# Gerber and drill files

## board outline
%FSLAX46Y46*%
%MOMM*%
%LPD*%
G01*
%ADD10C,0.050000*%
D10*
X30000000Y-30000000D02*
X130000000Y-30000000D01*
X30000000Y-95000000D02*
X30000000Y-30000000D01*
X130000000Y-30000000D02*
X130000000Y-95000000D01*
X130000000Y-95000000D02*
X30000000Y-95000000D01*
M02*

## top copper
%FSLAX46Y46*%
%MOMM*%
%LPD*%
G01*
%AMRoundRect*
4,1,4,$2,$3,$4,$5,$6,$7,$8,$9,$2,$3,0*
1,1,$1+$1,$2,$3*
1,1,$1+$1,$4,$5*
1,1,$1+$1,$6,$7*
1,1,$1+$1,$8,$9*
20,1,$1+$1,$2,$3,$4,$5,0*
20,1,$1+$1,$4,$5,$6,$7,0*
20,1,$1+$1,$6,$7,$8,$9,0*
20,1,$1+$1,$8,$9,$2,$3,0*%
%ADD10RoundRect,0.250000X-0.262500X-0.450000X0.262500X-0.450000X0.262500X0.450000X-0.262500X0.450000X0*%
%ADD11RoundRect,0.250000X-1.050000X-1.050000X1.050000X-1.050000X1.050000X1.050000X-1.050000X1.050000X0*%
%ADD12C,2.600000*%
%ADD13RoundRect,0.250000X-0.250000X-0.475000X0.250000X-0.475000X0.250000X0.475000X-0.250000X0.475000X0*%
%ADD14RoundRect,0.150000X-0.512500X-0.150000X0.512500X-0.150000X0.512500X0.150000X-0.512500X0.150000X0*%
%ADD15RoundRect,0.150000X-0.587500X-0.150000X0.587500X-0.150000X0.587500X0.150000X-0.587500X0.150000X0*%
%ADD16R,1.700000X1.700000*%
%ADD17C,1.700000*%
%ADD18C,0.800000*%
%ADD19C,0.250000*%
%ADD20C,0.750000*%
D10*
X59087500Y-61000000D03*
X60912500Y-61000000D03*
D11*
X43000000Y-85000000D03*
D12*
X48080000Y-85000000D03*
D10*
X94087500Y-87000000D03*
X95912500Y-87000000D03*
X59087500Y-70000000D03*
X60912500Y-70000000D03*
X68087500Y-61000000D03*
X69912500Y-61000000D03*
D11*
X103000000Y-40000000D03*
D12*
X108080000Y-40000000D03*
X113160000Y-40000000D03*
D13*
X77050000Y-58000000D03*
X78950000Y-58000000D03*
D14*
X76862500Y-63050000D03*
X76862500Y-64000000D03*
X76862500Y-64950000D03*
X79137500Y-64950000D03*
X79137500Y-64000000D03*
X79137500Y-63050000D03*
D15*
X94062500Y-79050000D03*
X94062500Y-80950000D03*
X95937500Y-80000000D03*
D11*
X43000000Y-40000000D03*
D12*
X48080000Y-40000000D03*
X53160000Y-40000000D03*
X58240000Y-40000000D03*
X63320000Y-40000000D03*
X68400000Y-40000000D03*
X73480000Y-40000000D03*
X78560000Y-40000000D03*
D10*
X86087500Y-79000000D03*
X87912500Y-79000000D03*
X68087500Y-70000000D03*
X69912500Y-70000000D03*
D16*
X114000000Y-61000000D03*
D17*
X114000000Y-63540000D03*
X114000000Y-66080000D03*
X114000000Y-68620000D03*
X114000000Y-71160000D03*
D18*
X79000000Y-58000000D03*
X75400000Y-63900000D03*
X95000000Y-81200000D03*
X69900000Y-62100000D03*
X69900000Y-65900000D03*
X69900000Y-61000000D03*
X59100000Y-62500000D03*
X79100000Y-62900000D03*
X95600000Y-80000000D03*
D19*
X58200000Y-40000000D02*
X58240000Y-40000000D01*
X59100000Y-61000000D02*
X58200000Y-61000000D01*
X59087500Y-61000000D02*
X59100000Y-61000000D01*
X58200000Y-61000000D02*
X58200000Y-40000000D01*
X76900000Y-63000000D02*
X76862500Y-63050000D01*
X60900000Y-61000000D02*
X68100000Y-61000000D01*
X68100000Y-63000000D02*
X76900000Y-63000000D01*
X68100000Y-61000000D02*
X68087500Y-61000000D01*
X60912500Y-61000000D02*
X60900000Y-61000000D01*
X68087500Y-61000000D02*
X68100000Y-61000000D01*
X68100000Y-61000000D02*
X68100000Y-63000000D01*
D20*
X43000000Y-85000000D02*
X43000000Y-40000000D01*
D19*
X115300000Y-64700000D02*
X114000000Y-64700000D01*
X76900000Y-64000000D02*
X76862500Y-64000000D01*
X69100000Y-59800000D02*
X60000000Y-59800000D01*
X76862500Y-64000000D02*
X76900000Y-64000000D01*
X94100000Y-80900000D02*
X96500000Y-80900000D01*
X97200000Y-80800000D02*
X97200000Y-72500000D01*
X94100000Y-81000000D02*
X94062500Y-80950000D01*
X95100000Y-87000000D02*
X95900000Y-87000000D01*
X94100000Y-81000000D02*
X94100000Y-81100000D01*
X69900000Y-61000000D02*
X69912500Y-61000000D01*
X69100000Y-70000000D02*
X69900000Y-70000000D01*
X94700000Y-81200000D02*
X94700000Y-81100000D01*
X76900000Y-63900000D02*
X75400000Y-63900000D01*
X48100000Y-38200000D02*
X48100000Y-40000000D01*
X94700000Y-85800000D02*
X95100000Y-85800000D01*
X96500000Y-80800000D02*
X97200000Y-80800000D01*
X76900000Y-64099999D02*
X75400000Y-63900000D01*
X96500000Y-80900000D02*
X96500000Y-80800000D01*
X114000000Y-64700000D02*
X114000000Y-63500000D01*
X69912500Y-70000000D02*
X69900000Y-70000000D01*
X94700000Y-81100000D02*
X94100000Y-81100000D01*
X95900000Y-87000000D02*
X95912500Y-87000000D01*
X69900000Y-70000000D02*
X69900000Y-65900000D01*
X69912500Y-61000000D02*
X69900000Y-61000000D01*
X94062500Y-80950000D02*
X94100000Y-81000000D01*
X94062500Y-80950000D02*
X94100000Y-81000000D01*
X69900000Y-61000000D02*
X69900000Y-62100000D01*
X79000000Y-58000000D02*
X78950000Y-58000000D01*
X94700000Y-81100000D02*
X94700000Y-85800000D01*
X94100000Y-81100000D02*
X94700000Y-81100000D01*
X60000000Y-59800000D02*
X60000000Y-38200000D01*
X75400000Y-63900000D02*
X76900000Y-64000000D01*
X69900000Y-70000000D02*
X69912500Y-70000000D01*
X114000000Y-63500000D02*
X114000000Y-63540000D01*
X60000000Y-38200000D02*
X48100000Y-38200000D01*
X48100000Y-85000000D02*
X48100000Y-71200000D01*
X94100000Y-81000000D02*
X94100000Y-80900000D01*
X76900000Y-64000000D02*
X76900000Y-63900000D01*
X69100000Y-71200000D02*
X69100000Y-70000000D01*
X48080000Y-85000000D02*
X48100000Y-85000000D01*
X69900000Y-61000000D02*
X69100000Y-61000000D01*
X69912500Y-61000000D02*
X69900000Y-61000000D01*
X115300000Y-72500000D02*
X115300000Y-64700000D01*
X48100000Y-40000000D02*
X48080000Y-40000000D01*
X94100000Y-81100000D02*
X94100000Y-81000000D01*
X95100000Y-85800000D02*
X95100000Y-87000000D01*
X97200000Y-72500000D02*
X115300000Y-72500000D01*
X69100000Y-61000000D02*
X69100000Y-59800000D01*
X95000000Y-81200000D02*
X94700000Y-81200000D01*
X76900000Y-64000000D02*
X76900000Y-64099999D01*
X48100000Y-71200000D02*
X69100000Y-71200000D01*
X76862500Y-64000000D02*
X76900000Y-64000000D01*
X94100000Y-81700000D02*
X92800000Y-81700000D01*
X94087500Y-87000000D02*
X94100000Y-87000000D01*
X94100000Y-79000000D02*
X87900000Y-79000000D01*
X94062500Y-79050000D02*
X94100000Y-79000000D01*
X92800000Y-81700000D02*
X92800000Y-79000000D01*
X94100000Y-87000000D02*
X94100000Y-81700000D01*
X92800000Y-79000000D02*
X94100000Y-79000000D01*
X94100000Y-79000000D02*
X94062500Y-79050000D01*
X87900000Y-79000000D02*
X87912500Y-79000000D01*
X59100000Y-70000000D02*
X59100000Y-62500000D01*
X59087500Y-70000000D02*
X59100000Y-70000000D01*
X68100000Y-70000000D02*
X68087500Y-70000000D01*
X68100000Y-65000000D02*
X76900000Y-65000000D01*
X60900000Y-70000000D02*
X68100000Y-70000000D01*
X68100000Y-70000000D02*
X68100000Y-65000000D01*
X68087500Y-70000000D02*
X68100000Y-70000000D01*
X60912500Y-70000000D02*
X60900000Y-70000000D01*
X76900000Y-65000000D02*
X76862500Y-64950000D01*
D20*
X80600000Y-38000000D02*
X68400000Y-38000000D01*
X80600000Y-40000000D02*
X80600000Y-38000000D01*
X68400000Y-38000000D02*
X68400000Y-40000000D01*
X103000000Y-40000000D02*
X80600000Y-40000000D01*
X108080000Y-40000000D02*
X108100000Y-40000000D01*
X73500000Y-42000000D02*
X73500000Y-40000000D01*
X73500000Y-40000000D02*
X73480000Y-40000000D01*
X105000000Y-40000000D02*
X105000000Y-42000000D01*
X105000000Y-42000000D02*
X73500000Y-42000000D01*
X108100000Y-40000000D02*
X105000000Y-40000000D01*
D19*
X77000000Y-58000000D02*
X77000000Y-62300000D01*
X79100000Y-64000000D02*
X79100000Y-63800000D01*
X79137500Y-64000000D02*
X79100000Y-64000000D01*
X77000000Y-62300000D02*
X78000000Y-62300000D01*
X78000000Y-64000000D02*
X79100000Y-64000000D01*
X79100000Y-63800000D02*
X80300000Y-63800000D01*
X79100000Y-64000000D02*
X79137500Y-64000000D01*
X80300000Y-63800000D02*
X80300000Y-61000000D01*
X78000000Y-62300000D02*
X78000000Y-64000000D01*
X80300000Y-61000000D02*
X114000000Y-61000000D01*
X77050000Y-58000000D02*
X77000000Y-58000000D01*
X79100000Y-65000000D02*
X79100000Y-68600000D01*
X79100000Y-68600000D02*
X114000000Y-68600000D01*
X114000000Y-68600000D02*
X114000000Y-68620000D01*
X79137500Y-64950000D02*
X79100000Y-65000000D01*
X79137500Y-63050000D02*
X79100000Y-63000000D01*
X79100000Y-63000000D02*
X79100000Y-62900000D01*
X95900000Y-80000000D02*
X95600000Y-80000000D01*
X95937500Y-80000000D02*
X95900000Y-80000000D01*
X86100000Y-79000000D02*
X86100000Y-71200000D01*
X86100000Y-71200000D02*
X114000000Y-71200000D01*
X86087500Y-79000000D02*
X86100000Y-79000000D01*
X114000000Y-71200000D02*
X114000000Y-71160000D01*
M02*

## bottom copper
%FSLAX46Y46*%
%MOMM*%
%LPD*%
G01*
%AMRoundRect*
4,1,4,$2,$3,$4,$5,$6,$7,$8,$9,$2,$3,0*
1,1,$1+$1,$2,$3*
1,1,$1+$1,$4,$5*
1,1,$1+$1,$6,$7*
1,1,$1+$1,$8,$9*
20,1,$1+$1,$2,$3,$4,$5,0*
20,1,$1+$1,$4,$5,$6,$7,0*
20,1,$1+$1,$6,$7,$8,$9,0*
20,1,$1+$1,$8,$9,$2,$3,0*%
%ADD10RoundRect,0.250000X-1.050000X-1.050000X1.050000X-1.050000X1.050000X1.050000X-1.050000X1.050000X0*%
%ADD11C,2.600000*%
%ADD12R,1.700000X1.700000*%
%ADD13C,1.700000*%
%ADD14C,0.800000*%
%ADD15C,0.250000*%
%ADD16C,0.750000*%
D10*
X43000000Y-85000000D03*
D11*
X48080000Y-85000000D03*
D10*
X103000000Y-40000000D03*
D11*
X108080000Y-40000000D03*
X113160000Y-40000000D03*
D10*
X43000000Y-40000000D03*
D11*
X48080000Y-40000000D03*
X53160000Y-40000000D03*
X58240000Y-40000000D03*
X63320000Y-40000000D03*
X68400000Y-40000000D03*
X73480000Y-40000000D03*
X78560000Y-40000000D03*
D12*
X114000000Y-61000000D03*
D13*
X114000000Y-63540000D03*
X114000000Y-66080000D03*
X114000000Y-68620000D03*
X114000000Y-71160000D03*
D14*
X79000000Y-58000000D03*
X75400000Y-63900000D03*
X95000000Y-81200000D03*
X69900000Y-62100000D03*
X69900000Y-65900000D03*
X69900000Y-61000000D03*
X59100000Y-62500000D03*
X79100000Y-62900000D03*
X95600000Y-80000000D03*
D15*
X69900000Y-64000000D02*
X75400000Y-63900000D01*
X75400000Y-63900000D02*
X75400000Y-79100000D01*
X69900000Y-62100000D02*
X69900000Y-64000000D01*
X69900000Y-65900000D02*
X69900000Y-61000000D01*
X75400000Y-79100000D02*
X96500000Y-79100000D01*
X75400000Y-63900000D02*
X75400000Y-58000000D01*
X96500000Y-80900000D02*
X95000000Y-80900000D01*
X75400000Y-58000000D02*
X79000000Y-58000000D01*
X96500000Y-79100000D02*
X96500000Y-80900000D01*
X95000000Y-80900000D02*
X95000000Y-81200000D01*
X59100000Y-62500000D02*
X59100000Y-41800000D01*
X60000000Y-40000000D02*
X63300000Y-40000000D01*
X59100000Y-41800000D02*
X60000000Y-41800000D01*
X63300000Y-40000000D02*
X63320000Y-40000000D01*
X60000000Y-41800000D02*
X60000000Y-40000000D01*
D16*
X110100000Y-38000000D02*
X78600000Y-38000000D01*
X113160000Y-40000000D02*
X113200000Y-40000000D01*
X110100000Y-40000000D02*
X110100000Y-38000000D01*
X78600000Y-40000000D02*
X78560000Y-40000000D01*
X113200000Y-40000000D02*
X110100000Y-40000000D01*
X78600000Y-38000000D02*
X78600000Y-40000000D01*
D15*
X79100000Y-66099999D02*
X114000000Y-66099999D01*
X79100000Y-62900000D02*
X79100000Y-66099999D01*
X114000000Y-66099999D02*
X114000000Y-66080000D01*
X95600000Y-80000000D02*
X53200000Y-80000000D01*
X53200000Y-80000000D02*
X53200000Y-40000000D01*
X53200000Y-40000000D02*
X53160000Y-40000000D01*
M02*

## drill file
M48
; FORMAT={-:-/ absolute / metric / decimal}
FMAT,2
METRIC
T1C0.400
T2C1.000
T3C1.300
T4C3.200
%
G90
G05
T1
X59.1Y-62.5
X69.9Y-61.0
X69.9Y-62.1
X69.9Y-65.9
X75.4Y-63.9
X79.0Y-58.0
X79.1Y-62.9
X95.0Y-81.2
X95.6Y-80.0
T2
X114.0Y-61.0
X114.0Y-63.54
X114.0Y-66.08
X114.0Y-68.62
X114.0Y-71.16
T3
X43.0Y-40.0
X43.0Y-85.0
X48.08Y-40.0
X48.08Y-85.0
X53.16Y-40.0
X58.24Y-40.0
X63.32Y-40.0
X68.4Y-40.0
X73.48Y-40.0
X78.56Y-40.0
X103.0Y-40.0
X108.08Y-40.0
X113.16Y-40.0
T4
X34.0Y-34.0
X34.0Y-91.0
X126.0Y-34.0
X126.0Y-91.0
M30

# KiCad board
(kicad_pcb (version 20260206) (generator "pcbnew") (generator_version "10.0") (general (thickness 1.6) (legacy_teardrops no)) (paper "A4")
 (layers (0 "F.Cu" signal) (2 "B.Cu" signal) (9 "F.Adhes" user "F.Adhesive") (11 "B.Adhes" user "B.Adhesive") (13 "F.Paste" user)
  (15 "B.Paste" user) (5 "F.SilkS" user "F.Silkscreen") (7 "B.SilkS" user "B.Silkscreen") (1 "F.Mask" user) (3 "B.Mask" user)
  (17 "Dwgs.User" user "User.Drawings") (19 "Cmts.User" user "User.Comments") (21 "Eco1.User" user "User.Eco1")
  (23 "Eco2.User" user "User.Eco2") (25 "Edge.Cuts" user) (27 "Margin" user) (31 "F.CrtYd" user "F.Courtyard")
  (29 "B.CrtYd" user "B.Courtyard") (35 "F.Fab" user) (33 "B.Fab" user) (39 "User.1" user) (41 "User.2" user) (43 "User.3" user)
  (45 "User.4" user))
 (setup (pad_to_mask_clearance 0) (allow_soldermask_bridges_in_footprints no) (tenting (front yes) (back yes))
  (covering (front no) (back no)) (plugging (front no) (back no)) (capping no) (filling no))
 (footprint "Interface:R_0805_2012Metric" (layer "F.Cu") (at 60 61)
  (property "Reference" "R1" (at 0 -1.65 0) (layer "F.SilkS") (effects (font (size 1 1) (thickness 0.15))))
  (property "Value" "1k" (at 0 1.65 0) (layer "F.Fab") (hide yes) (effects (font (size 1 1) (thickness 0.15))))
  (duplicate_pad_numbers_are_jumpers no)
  (pad "1" smd roundrect (at -0.9125 0) (size 1.025 1.4) (layers "F.Cu" "F.Mask" "F.Paste") (roundrect_rratio 0.243902) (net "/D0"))
  (pad "2" smd roundrect (at 0.9125 0) (size 1.025 1.4) (layers "F.Cu" "F.Mask" "F.Paste") (roundrect_rratio 0.243902) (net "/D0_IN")))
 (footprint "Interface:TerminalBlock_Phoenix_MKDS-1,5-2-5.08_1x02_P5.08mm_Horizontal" (layer "F.Cu") (at 43 85)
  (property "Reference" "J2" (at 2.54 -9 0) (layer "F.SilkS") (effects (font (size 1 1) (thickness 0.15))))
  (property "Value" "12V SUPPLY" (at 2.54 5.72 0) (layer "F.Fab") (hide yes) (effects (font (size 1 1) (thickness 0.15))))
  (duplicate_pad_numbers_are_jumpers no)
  (pad "1" thru_hole roundrect (at 0 0) (size 2.6 2.6) (drill 1.3) (layers "*.Cu" "*.Mask") (remove_unused_layers no)
   (roundrect_rratio 0.096154) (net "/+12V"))
  (pad "2" thru_hole circle (at 5.08 0) (size 2.6 2.6) (drill 1.3) (layers "*.Cu" "*.Mask") (remove_unused_layers no) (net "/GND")))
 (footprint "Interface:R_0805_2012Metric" (layer "F.Cu") (at 95 87)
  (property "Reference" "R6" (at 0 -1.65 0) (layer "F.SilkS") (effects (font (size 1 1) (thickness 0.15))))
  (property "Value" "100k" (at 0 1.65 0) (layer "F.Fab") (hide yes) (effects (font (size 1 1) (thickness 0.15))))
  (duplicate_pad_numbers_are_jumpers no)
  (pad "1" smd roundrect (at -0.9125 0) (size 1.025 1.4) (layers "F.Cu" "F.Mask" "F.Paste") (roundrect_rratio 0.243902) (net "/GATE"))
  (pad "2" smd roundrect (at 0.9125 0) (size 1.025 1.4) (layers "F.Cu" "F.Mask" "F.Paste") (roundrect_rratio 0.243902) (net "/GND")))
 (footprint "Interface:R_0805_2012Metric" (layer "F.Cu") (at 60 70)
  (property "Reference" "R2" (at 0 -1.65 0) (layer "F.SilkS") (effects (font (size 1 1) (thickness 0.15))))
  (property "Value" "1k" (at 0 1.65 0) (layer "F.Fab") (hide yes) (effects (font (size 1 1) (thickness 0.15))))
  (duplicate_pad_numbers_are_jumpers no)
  (pad "1" smd roundrect (at -0.9125 0) (size 1.025 1.4) (layers "F.Cu" "F.Mask" "F.Paste") (roundrect_rratio 0.243902) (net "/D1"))
  (pad "2" smd roundrect (at 0.9125 0) (size 1.025 1.4) (layers "F.Cu" "F.Mask" "F.Paste") (roundrect_rratio 0.243902) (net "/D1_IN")))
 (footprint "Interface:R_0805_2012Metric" (layer "F.Cu") (at 69 61)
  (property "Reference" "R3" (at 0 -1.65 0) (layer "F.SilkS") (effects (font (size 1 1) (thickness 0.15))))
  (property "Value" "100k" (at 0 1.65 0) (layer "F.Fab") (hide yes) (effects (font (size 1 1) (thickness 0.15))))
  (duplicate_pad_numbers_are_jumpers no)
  (pad "1" smd roundrect (at -0.9125 0) (size 1.025 1.4) (layers "F.Cu" "F.Mask" "F.Paste") (roundrect_rratio 0.243902) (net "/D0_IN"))
  (pad "2" smd roundrect (at 0.9125 0) (size 1.025 1.4) (layers "F.Cu" "F.Mask" "F.Paste") (roundrect_rratio 0.243902) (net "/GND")))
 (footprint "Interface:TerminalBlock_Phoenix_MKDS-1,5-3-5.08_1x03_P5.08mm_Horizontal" (layer "F.Cu") (at 103 40)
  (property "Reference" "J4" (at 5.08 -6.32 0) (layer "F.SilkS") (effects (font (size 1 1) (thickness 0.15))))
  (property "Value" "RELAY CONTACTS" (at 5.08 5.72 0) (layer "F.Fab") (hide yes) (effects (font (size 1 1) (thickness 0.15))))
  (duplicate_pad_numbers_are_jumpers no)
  (pad "1" thru_hole roundrect (at 0 0) (size 2.6 2.6) (drill 1.3) (layers "*.Cu" "*.Mask") (remove_unused_layers no)
   (roundrect_rratio 0.096154) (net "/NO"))
  (pad "2" thru_hole circle (at 5.08 0) (size 2.6 2.6) (drill 1.3) (layers "*.Cu" "*.Mask") (remove_unused_layers no) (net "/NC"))
  (pad "3" thru_hole circle (at 10.16 0) (size 2.6 2.6) (drill 1.3) (layers "*.Cu" "*.Mask") (remove_unused_layers no) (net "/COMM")))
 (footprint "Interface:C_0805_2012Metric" (layer "F.Cu") (at 78 58)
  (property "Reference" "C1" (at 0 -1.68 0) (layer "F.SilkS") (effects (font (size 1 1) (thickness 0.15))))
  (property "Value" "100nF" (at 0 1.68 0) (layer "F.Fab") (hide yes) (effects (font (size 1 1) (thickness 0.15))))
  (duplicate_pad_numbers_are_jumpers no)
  (pad "1" smd roundrect (at -0.95 0) (size 1 1.45) (layers "F.Cu" "F.Mask" "F.Paste") (roundrect_rratio 0.25) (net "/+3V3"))
  (pad "2" smd roundrect (at 0.95 0) (size 1 1.45) (layers "F.Cu" "F.Mask" "F.Paste") (roundrect_rratio 0.25) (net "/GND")))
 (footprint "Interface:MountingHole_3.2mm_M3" (layer "F.Cu") (at 34 91)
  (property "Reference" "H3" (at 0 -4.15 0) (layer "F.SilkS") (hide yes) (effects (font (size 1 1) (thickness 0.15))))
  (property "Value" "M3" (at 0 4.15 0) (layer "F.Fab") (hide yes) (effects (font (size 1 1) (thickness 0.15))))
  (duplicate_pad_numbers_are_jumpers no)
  (pad "" np_thru_hole circle (at 0 0) (size 3.2 3.2) (drill 3.2) (layers "*.Cu" "*.Mask")))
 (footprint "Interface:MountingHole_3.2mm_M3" (layer "F.Cu") (at 126 91)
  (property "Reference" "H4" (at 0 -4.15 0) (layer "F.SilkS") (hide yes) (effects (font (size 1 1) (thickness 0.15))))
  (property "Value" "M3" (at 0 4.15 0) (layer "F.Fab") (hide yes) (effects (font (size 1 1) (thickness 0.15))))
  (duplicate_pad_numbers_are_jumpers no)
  (pad "" np_thru_hole circle (at 0 0) (size 3.2 3.2) (drill 3.2) (layers "*.Cu" "*.Mask")))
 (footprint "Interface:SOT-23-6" (layer "F.Cu") (at 78 64)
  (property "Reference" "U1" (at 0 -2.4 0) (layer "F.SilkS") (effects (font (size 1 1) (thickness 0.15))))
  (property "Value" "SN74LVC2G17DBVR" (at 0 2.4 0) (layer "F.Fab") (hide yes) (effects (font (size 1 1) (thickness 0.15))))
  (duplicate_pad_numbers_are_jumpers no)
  (pad "1" smd roundrect (at -1.1375 -0.95) (size 1.325 0.6) (layers "F.Cu" "F.Mask" "F.Paste") (roundrect_rratio 0.25) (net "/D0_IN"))
  (pad "2" smd roundrect (at -1.1375 0) (size 1.325 0.6) (layers "F.Cu" "F.Mask" "F.Paste") (roundrect_rratio 0.25) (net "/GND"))
  (pad "3" smd roundrect (at -1.1375 0.95) (size 1.325 0.6) (layers "F.Cu" "F.Mask" "F.Paste") (roundrect_rratio 0.25) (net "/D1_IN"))
  (pad "4" smd roundrect (at 1.1375 0.95) (size 1.325 0.6) (layers "F.Cu" "F.Mask" "F.Paste") (roundrect_rratio 0.25) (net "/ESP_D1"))
  (pad "5" smd roundrect (at 1.1375 0) (size 1.325 0.6) (layers "F.Cu" "F.Mask" "F.Paste") (roundrect_rratio 0.25) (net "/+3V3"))
  (pad "6" smd roundrect (at 1.1375 -0.95) (size 1.325 0.6) (layers "F.Cu" "F.Mask" "F.Paste") (roundrect_rratio 0.25) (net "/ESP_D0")))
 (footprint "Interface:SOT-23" (layer "F.Cu") (at 95 80)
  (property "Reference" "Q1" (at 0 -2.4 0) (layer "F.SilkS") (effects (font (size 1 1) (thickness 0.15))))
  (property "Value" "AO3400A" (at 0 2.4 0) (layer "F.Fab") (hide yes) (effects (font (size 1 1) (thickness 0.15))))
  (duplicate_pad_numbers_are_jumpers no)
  (pad "1" smd roundrect (at -0.9375 -0.95) (size 1.475 0.6) (layers "F.Cu" "F.Mask" "F.Paste") (roundrect_rratio 0.25) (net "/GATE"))
  (pad "2" smd roundrect (at -0.9375 0.95) (size 1.475 0.6) (layers "F.Cu" "F.Mask" "F.Paste") (roundrect_rratio 0.25) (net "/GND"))
  (pad "3" smd roundrect (at 0.9375 0) (size 1.475 0.6) (layers "F.Cu" "F.Mask" "F.Paste") (roundrect_rratio 0.25) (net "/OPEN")))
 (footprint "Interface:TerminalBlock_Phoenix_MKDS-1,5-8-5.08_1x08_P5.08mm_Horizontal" (layer "F.Cu") (at 43 40)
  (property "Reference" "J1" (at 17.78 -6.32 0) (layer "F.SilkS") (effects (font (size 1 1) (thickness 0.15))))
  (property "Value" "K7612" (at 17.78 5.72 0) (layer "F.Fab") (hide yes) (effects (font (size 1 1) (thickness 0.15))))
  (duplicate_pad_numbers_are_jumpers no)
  (pad "1" thru_hole roundrect (at 0 0) (size 2.6 2.6) (drill 1.3) (layers "*.Cu" "*.Mask") (remove_unused_layers no)
   (roundrect_rratio 0.096154) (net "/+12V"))
  (pad "2" thru_hole circle (at 5.08 0) (size 2.6 2.6) (drill 1.3) (layers "*.Cu" "*.Mask") (remove_unused_layers no) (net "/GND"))
  (pad "3" thru_hole circle (at 10.16 0) (size 2.6 2.6) (drill 1.3) (layers "*.Cu" "*.Mask") (remove_unused_layers no) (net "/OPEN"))
  (pad "4" thru_hole circle (at 15.24 0) (size 2.6 2.6) (drill 1.3) (layers "*.Cu" "*.Mask") (remove_unused_layers no) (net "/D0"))
  (pad "5" thru_hole circle (at 20.32 0) (size 2.6 2.6) (drill 1.3) (layers "*.Cu" "*.Mask") (remove_unused_layers no) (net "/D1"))
  (pad "6" thru_hole circle (at 25.4 0) (size 2.6 2.6) (drill 1.3) (layers "*.Cu" "*.Mask") (remove_unused_layers no) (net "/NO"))
  (pad "7" thru_hole circle (at 30.48 0) (size 2.6 2.6) (drill 1.3) (layers "*.Cu" "*.Mask") (remove_unused_layers no) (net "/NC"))
  (pad "8" thru_hole circle (at 35.56 0) (size 2.6 2.6) (drill 1.3) (layers "*.Cu" "*.Mask") (remove_unused_layers no) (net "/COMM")))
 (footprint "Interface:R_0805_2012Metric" (layer "F.Cu") (at 87 79)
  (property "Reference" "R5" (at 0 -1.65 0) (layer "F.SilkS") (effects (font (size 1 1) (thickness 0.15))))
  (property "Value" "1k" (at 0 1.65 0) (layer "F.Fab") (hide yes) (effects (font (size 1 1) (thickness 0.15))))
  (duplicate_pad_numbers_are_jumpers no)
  (pad "1" smd roundrect (at -0.9125 0) (size 1.025 1.4) (layers "F.Cu" "F.Mask" "F.Paste") (roundrect_rratio 0.243902) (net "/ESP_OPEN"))
  (pad "2" smd roundrect (at 0.9125 0) (size 1.025 1.4) (layers "F.Cu" "F.Mask" "F.Paste") (roundrect_rratio 0.243902) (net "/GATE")))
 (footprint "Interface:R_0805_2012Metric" (layer "F.Cu") (at 69 70)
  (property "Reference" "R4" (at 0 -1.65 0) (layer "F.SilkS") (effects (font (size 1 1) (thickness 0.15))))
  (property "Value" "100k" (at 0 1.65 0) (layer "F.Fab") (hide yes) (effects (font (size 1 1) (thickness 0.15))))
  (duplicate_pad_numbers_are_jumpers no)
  (pad "1" smd roundrect (at -0.9125 0) (size 1.025 1.4) (layers "F.Cu" "F.Mask" "F.Paste") (roundrect_rratio 0.243902) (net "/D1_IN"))
  (pad "2" smd roundrect (at 0.9125 0) (size 1.025 1.4) (layers "F.Cu" "F.Mask" "F.Paste") (roundrect_rratio 0.243902) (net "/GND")))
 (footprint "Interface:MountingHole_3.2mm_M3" (layer "F.Cu") (at 126 34)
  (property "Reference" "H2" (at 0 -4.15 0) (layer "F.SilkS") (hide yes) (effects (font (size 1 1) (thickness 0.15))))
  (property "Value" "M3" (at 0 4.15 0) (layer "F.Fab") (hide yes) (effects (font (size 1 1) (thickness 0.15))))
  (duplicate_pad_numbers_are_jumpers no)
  (pad "" np_thru_hole circle (at 0 0) (size 3.2 3.2) (drill 3.2) (layers "*.Cu" "*.Mask")))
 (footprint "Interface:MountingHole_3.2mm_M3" (layer "F.Cu") (at 34 34)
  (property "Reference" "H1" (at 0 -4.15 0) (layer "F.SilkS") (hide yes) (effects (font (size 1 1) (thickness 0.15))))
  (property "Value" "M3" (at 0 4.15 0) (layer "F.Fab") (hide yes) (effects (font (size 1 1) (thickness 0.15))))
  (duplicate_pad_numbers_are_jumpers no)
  (pad "" np_thru_hole circle (at 0 0) (size 3.2 3.2) (drill 3.2) (layers "*.Cu" "*.Mask")))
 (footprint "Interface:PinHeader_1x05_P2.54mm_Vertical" (layer "F.Cu") (at 114 61)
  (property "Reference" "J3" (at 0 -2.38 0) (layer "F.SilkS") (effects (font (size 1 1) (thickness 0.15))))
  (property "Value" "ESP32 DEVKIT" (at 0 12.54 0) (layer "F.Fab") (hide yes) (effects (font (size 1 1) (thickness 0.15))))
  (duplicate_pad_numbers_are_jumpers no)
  (pad "1" thru_hole rect (at 0 0) (size 1.7 1.7) (drill 1) (layers "*.Cu" "*.Mask") (remove_unused_layers no) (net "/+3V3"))
  (pad "2" thru_hole circle (at 0 2.54) (size 1.7 1.7) (drill 1) (layers "*.Cu" "*.Mask") (remove_unused_layers no) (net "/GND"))
  (pad "3" thru_hole circle (at 0 5.08) (size 1.7 1.7) (drill 1) (layers "*.Cu" "*.Mask") (remove_unused_layers no) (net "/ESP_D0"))
  (pad "4" thru_hole circle (at 0 7.62) (size 1.7 1.7) (drill 1) (layers "*.Cu" "*.Mask") (remove_unused_layers no) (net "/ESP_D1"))
  (pad "5" thru_hole circle (at 0 10.16) (size 1.7 1.7) (drill 1) (layers "*.Cu" "*.Mask") (remove_unused_layers no) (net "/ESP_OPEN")))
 (gr_line (start 30 30) (end 130 30) (stroke (width 0.05) (type default)) (layer "Edge.Cuts"))
 (gr_line (start 30 95) (end 30 30) (stroke (width 0.05) (type default)) (layer "Edge.Cuts"))
 (gr_line (start 130 30) (end 130 95) (stroke (width 0.05) (type default)) (layer "Edge.Cuts"))
 (gr_line (start 130 95) (end 30 95) (stroke (width 0.05) (type default)) (layer "Edge.Cuts"))
 (segment (start 58.2 40) (end 58.24 40) (width 0.25) (layer "F.Cu") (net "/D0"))
 (segment (start 59.1 61) (end 58.2 61) (width 0.25) (layer "F.Cu") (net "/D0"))
 (segment (start 59.0875 61) (end 59.1 61) (width 0.25) (layer "F.Cu") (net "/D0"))
 (segment (start 58.2 61) (end 58.2 40) (width 0.25) (layer "F.Cu") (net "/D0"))
 (segment (start 76.9 63) (end 76.8625 63.05) (width 0.25) (layer "F.Cu") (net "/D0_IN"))
 (segment (start 60.9 61) (end 68.1 61) (width 0.25) (layer "F.Cu") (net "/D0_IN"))
 (segment (start 68.1 63) (end 76.9 63) (width 0.25) (layer "F.Cu") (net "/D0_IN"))
 (segment (start 68.1 61) (end 68.0875 61) (width 0.25) (layer "F.Cu") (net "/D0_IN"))
 (segment (start 60.9125 61) (end 60.9 61) (width 0.25) (layer "F.Cu") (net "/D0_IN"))
 (segment (start 68.0875 61) (end 68.1 61) (width 0.25) (layer "F.Cu") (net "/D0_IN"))
 (segment (start 68.1 61) (end 68.1 63) (width 0.25) (layer "F.Cu") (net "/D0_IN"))
 (segment (start 43 85) (end 43 40) (width 0.75) (layer "F.Cu") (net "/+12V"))
 (segment (start 115.3 64.7) (end 114 64.7) (width 0.25) (layer "F.Cu") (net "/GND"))
 (segment (start 76.9 64) (end 76.8625 64) (width 0.25) (layer "F.Cu") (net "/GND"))
 (segment (start 69.1 59.8) (end 60 59.8) (width 0.25) (layer "F.Cu") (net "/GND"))
 (segment (start 76.8625 64) (end 76.9 64) (width 0.25) (layer "F.Cu") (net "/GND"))
 (segment (start 94.1 80.9) (end 96.5 80.9) (width 0.25) (layer "F.Cu") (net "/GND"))
 (segment (start 97.2 80.8) (end 97.2 72.5) (width 0.25) (layer "F.Cu") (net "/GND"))
 (segment (start 94.1 81) (end 94.0625 80.95) (width 0.25) (layer "F.Cu") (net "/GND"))
 (segment (start 95.1 87) (end 95.9 87) (width 0.25) (layer "F.Cu") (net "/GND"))
 (segment (start 94.1 81) (end 94.1 81.1) (width 0.25) (layer "F.Cu") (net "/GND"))
 (segment (start 69.9 61) (end 69.9125 61) (width 0.25) (layer "F.Cu") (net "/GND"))
 (segment (start 69.1 70) (end 69.9 70) (width 0.25) (layer "F.Cu") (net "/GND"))
 (segment (start 94.7 81.2) (end 94.7 81.1) (width 0.25) (layer "F.Cu") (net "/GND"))
 (segment (start 76.9 63.9) (end 75.4 63.9) (width 0.25) (layer "F.Cu") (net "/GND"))
 (segment (start 48.1 38.2) (end 48.1 40) (width 0.25) (layer "F.Cu") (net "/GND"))
 (segment (start 94.7 85.8) (end 95.1 85.8) (width 0.25) (layer "F.Cu") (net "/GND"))
 (segment (start 96.5 80.8) (end 97.2 80.8) (width 0.25) (layer "F.Cu") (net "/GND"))
 (segment (start 76.9 64.099999) (end 75.4 63.9) (width 0.25) (layer "F.Cu") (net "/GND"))
 (segment (start 96.5 80.9) (end 96.5 80.8) (width 0.25) (layer "F.Cu") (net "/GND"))
 (segment (start 114 64.7) (end 114 63.5) (width 0.25) (layer "F.Cu") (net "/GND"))
 (segment (start 69.9125 70) (end 69.9 70) (width 0.25) (layer "F.Cu") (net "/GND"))
 (segment (start 94.7 81.1) (end 94.1 81.1) (width 0.25) (layer "F.Cu") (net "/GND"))
 (segment (start 95.9 87) (end 95.9125 87) (width 0.25) (layer "F.Cu") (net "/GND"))
 (segment (start 69.9 70) (end 69.9 65.9) (width 0.25) (layer "F.Cu") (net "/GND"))
 (segment (start 69.9125 61) (end 69.9 61) (width 0.25) (layer "F.Cu") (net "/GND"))
 (segment (start 94.0625 80.95) (end 94.1 81) (width 0.25) (layer "F.Cu") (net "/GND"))
 (segment (start 94.0625 80.95) (end 94.1 81) (width 0.25) (layer "F.Cu") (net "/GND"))
 (segment (start 69.9 61) (end 69.9 62.1) (width 0.25) (layer "F.Cu") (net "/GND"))
 (segment (start 79 58) (end 78.95 58) (width 0.25) (layer "F.Cu") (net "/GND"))
 (segment (start 94.7 81.1) (end 94.7 85.8) (width 0.25) (layer "F.Cu") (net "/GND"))
 (segment (start 94.1 81.1) (end 94.7 81.1) (width 0.25) (layer "F.Cu") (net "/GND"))
 (segment (start 60 59.8) (end 60 38.2) (width 0.25) (layer "F.Cu") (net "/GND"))
 (segment (start 75.4 63.9) (end 76.9 64) (width 0.25) (layer "F.Cu") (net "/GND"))
 (segment (start 69.9 70) (end 69.9125 70) (width 0.25) (layer "F.Cu") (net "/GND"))
 (segment (start 114 63.5) (end 114 63.54) (width 0.25) (layer "F.Cu") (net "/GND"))
 (segment (start 60 38.2) (end 48.1 38.2) (width 0.25) (layer "F.Cu") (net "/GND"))
 (segment (start 48.1 85) (end 48.1 71.2) (width 0.25) (layer "F.Cu") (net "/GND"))
 (segment (start 94.1 81) (end 94.1 80.9) (width 0.25) (layer "F.Cu") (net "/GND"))
 (segment (start 76.9 64) (end 76.9 63.9) (width 0.25) (layer "F.Cu") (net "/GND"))
 (segment (start 69.1 71.2) (end 69.1 70) (width 0.25) (layer "F.Cu") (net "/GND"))
 (segment (start 48.08 85) (end 48.1 85) (width 0.25) (layer "F.Cu") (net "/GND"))
 (segment (start 69.9 61) (end 69.1 61) (width 0.25) (layer "F.Cu") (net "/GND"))
 (segment (start 69.9125 61) (end 69.9 61) (width 0.25) (layer "F.Cu") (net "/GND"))
 (segment (start 115.3 72.5) (end 115.3 64.7) (width 0.25) (layer "F.Cu") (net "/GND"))
 (segment (start 48.1 40) (end 48.08 40) (width 0.25) (layer "F.Cu") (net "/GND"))
 (segment (start 94.1 81.1) (end 94.1 81) (width 0.25) (layer "F.Cu") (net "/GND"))
 (segment (start 95.1 85.8) (end 95.1 87) (width 0.25) (layer "F.Cu") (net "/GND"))
 (segment (start 97.2 72.5) (end 115.3 72.5) (width 0.25) (layer "F.Cu") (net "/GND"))
 (segment (start 69.1 61) (end 69.1 59.8) (width 0.25) (layer "F.Cu") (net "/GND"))
 (segment (start 95 81.2) (end 94.7 81.2) (width 0.25) (layer "F.Cu") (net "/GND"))
 (segment (start 76.9 64) (end 76.9 64.099999) (width 0.25) (layer "F.Cu") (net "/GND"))
 (segment (start 48.1 71.2) (end 69.1 71.2) (width 0.25) (layer "F.Cu") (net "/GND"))
 (segment (start 76.8625 64) (end 76.9 64) (width 0.25) (layer "F.Cu") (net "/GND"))
 (via (at 79 58) (size 0.8) (drill 0.4) (layers "F.Cu" "B.Cu") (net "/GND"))
 (via (at 75.4 63.9) (size 0.8) (drill 0.4) (layers "F.Cu" "B.Cu") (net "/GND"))
 (via (at 95 81.2) (size 0.8) (drill 0.4) (layers "F.Cu" "B.Cu") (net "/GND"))
 (via (at 69.9 62.1) (size 0.8) (drill 0.4) (layers "F.Cu" "B.Cu") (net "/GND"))
 (via (at 69.9 65.9) (size 0.8) (drill 0.4) (layers "F.Cu" "B.Cu") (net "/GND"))
 (via (at 69.9 61) (size 0.8) (drill 0.4) (layers "F.Cu" "B.Cu") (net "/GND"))
 (segment (start 69.9 64) (end 75.4 63.9) (width 0.25) (layer "B.Cu") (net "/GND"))
 (segment (start 75.4 63.9) (end 75.4 79.1) (width 0.25) (layer "B.Cu") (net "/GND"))
 (segment (start 69.9 62.1) (end 69.9 64) (width 0.25) (layer "B.Cu") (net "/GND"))
 (segment (start 69.9 65.9) (end 69.9 61) (width 0.25) (layer "B.Cu") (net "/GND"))
 (segment (start 75.4 79.1) (end 96.5 79.1) (width 0.25) (layer "B.Cu") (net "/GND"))
 (segment (start 75.4 63.9) (end 75.4 58) (width 0.25) (layer "B.Cu") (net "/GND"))
 (segment (start 96.5 80.9) (end 95 80.9) (width 0.25) (layer "B.Cu") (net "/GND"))
 (segment (start 75.4 58) (end 79 58) (width 0.25) (layer "B.Cu") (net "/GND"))
 (segment (start 96.5 79.1) (end 96.5 80.9) (width 0.25) (layer "B.Cu") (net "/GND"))
 (segment (start 95 80.9) (end 95 81.2) (width 0.25) (layer "B.Cu") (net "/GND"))
 (segment (start 94.1 81.7) (end 92.8 81.7) (width 0.25) (layer "F.Cu") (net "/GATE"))
 (segment (start 94.0875 87) (end 94.1 87) (width 0.25) (layer "F.Cu") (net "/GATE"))
 (segment (start 94.1 79) (end 87.9 79) (width 0.25) (layer "F.Cu") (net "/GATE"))
 (segment (start 94.0625 79.05) (end 94.1 79) (width 0.25) (layer "F.Cu") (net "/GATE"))
 (segment (start 92.8 81.7) (end 92.8 79) (width 0.25) (layer "F.Cu") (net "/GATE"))
 (segment (start 94.1 87) (end 94.1 81.7) (width 0.25) (layer "F.Cu") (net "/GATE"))
 (segment (start 92.8 79) (end 94.1 79) (width 0.25) (layer "F.Cu") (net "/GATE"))
 (segment (start 94.1 79) (end 94.0625 79.05) (width 0.25) (layer "F.Cu") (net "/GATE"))
 (segment (start 87.9 79) (end 87.9125 79) (width 0.25) (layer "F.Cu") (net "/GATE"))
 (segment (start 59.1 70) (end 59.1 62.5) (width 0.25) (layer "F.Cu") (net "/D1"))
 (segment (start 59.0875 70) (end 59.1 70) (width 0.25) (layer "F.Cu") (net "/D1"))
 (via (at 59.1 62.5) (size 0.8) (drill 0.4) (layers "F.Cu" "B.Cu") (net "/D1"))
 (segment (start 59.1 62.5) (end 59.1 41.8) (width 0.25) (layer "B.Cu") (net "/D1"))
 (segment (start 60 40) (end 63.3 40) (width 0.25) (layer "B.Cu") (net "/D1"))
 (segment (start 59.1 41.8) (end 60 41.8) (width 0.25) (layer "B.Cu") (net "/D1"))
 (segment (start 63.3 40) (end 63.32 40) (width 0.25) (layer "B.Cu") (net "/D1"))
 (segment (start 60 41.8) (end 60 40) (width 0.25) (layer "B.Cu") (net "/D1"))
 (segment (start 68.1 70) (end 68.0875 70) (width 0.25) (layer "F.Cu") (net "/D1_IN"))
 (segment (start 68.1 65) (end 76.9 65) (width 0.25) (layer "F.Cu") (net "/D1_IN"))
 (segment (start 60.9 70) (end 68.1 70) (width 0.25) (layer "F.Cu") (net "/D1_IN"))
 (segment (start 68.1 70) (end 68.1 65) (width 0.25) (layer "F.Cu") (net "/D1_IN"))
 (segment (start 68.0875 70) (end 68.1 70) (width 0.25) (layer "F.Cu") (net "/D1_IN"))
 (segment (start 60.9125 70) (end 60.9 70) (width 0.25) (layer "F.Cu") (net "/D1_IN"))
 (segment (start 76.9 65) (end 76.8625 64.95) (width 0.25) (layer "F.Cu") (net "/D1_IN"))
 (segment (start 80.6 38) (end 68.4 38) (width 0.75) (layer "F.Cu") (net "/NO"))
 (segment (start 80.6 40) (end 80.6 38) (width 0.75) (layer "F.Cu") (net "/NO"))
 (segment (start 68.4 38) (end 68.4 40) (width 0.75) (layer "F.Cu") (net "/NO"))
 (segment (start 103 40) (end 80.6 40) (width 0.75) (layer "F.Cu") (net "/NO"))
 (segment (start 108.08 40) (end 108.1 40) (width 0.75) (layer "F.Cu") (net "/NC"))
 (segment (start 73.5 42) (end 73.5 40) (width 0.75) (layer "F.Cu") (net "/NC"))
 (segment (start 73.5 40) (end 73.48 40) (width 0.75) (layer "F.Cu") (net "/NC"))
 (segment (start 105 40) (end 105 42) (width 0.75) (layer "F.Cu") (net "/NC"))
 (segment (start 105 42) (end 73.5 42) (width 0.75) (layer "F.Cu") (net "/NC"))
 (segment (start 108.1 40) (end 105 40) (width 0.75) (layer "F.Cu") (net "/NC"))
 (segment (start 110.1 38) (end 78.6 38) (width 0.75) (layer "B.Cu") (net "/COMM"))
 (segment (start 113.16 40) (end 113.2 40) (width 0.75) (layer "B.Cu") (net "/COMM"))
 (segment (start 110.1 40) (end 110.1 38) (width 0.75) (layer "B.Cu") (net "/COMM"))
 (segment (start 78.6 40) (end 78.56 40) (width 0.75) (layer "B.Cu") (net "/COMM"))
 (segment (start 113.2 40) (end 110.1 40) (width 0.75) (layer "B.Cu") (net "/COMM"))
 (segment (start 78.6 38) (end 78.6 40) (width 0.75) (layer "B.Cu") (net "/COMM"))
 (segment (start 77 58) (end 77 62.3) (width 0.25) (layer "F.Cu") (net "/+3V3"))
 (segment (start 79.1 64) (end 79.1 63.8) (width 0.25) (layer "F.Cu") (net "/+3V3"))
 (segment (start 79.1375 64) (end 79.1 64) (width 0.25) (layer "F.Cu") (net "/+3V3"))
 (segment (start 77 62.3) (end 78 62.3) (width 0.25) (layer "F.Cu") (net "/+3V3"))
 (segment (start 78 64) (end 79.1 64) (width 0.25) (layer "F.Cu") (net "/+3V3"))
 (segment (start 79.1 63.8) (end 80.3 63.8) (width 0.25) (layer "F.Cu") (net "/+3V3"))
 (segment (start 79.1 64) (end 79.1375 64) (width 0.25) (layer "F.Cu") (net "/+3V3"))
 (segment (start 80.3 63.8) (end 80.3 61) (width 0.25) (layer "F.Cu") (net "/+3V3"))
 (segment (start 78 62.3) (end 78 64) (width 0.25) (layer "F.Cu") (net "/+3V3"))
 (segment (start 80.3 61) (end 114 61) (width 0.25) (layer "F.Cu") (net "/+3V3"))
 (segment (start 77.05 58) (end 77 58) (width 0.25) (layer "F.Cu") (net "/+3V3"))
 (segment (start 79.1 65) (end 79.1 68.6) (width 0.25) (layer "F.Cu") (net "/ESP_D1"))
 (segment (start 79.1 68.6) (end 114 68.6) (width 0.25) (layer "F.Cu") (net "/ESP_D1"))
 (segment (start 114 68.6) (end 114 68.62) (width 0.25) (layer "F.Cu") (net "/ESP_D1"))
 (segment (start 79.1375 64.95) (end 79.1 65) (width 0.25) (layer "F.Cu") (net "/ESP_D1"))
 (segment (start 79.1375 63.05) (end 79.1 63) (width 0.25) (layer "F.Cu") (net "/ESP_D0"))
 (segment (start 79.1 63) (end 79.1 62.9) (width 0.25) (layer "F.Cu") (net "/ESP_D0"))
 (via (at 79.1 62.9) (size 0.8) (drill 0.4) (layers "F.Cu" "B.Cu") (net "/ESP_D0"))
 (segment (start 79.1 66.099999) (end 114 66.099999) (width 0.25) (layer "B.Cu") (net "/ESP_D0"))
 (segment (start 79.1 62.9) (end 79.1 66.099999) (width 0.25) (layer "B.Cu") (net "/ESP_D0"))
 (segment (start 114 66.099999) (end 114 66.08) (width 0.25) (layer "B.Cu") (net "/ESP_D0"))
 (segment (start 95.9 80) (end 95.6 80) (width 0.25) (layer "F.Cu") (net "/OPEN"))
 (segment (start 95.9375 80) (end 95.9 80) (width 0.25) (layer "F.Cu") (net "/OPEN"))
 (via (at 95.6 80) (size 0.8) (drill 0.4) (layers "F.Cu" "B.Cu") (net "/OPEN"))
 (segment (start 95.6 80) (end 53.2 80) (width 0.25) (layer "B.Cu") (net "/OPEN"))
 (segment (start 53.2 80) (end 53.2 40) (width 0.25) (layer "B.Cu") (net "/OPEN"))
 (segment (start 53.2 40) (end 53.16 40) (width 0.25) (layer "B.Cu") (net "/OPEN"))
 (segment (start 86.1 79) (end 86.1 71.2) (width 0.25) (layer "F.Cu") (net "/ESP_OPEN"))
 (segment (start 86.1 71.2) (end 114 71.2) (width 0.25) (layer "F.Cu") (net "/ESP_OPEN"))
 (segment (start 86.0875 79) (end 86.1 79) (width 0.25) (layer "F.Cu") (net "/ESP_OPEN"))
 (segment (start 114 71.2) (end 114 71.16) (width 0.25) (layer "F.Cu") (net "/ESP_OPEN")))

